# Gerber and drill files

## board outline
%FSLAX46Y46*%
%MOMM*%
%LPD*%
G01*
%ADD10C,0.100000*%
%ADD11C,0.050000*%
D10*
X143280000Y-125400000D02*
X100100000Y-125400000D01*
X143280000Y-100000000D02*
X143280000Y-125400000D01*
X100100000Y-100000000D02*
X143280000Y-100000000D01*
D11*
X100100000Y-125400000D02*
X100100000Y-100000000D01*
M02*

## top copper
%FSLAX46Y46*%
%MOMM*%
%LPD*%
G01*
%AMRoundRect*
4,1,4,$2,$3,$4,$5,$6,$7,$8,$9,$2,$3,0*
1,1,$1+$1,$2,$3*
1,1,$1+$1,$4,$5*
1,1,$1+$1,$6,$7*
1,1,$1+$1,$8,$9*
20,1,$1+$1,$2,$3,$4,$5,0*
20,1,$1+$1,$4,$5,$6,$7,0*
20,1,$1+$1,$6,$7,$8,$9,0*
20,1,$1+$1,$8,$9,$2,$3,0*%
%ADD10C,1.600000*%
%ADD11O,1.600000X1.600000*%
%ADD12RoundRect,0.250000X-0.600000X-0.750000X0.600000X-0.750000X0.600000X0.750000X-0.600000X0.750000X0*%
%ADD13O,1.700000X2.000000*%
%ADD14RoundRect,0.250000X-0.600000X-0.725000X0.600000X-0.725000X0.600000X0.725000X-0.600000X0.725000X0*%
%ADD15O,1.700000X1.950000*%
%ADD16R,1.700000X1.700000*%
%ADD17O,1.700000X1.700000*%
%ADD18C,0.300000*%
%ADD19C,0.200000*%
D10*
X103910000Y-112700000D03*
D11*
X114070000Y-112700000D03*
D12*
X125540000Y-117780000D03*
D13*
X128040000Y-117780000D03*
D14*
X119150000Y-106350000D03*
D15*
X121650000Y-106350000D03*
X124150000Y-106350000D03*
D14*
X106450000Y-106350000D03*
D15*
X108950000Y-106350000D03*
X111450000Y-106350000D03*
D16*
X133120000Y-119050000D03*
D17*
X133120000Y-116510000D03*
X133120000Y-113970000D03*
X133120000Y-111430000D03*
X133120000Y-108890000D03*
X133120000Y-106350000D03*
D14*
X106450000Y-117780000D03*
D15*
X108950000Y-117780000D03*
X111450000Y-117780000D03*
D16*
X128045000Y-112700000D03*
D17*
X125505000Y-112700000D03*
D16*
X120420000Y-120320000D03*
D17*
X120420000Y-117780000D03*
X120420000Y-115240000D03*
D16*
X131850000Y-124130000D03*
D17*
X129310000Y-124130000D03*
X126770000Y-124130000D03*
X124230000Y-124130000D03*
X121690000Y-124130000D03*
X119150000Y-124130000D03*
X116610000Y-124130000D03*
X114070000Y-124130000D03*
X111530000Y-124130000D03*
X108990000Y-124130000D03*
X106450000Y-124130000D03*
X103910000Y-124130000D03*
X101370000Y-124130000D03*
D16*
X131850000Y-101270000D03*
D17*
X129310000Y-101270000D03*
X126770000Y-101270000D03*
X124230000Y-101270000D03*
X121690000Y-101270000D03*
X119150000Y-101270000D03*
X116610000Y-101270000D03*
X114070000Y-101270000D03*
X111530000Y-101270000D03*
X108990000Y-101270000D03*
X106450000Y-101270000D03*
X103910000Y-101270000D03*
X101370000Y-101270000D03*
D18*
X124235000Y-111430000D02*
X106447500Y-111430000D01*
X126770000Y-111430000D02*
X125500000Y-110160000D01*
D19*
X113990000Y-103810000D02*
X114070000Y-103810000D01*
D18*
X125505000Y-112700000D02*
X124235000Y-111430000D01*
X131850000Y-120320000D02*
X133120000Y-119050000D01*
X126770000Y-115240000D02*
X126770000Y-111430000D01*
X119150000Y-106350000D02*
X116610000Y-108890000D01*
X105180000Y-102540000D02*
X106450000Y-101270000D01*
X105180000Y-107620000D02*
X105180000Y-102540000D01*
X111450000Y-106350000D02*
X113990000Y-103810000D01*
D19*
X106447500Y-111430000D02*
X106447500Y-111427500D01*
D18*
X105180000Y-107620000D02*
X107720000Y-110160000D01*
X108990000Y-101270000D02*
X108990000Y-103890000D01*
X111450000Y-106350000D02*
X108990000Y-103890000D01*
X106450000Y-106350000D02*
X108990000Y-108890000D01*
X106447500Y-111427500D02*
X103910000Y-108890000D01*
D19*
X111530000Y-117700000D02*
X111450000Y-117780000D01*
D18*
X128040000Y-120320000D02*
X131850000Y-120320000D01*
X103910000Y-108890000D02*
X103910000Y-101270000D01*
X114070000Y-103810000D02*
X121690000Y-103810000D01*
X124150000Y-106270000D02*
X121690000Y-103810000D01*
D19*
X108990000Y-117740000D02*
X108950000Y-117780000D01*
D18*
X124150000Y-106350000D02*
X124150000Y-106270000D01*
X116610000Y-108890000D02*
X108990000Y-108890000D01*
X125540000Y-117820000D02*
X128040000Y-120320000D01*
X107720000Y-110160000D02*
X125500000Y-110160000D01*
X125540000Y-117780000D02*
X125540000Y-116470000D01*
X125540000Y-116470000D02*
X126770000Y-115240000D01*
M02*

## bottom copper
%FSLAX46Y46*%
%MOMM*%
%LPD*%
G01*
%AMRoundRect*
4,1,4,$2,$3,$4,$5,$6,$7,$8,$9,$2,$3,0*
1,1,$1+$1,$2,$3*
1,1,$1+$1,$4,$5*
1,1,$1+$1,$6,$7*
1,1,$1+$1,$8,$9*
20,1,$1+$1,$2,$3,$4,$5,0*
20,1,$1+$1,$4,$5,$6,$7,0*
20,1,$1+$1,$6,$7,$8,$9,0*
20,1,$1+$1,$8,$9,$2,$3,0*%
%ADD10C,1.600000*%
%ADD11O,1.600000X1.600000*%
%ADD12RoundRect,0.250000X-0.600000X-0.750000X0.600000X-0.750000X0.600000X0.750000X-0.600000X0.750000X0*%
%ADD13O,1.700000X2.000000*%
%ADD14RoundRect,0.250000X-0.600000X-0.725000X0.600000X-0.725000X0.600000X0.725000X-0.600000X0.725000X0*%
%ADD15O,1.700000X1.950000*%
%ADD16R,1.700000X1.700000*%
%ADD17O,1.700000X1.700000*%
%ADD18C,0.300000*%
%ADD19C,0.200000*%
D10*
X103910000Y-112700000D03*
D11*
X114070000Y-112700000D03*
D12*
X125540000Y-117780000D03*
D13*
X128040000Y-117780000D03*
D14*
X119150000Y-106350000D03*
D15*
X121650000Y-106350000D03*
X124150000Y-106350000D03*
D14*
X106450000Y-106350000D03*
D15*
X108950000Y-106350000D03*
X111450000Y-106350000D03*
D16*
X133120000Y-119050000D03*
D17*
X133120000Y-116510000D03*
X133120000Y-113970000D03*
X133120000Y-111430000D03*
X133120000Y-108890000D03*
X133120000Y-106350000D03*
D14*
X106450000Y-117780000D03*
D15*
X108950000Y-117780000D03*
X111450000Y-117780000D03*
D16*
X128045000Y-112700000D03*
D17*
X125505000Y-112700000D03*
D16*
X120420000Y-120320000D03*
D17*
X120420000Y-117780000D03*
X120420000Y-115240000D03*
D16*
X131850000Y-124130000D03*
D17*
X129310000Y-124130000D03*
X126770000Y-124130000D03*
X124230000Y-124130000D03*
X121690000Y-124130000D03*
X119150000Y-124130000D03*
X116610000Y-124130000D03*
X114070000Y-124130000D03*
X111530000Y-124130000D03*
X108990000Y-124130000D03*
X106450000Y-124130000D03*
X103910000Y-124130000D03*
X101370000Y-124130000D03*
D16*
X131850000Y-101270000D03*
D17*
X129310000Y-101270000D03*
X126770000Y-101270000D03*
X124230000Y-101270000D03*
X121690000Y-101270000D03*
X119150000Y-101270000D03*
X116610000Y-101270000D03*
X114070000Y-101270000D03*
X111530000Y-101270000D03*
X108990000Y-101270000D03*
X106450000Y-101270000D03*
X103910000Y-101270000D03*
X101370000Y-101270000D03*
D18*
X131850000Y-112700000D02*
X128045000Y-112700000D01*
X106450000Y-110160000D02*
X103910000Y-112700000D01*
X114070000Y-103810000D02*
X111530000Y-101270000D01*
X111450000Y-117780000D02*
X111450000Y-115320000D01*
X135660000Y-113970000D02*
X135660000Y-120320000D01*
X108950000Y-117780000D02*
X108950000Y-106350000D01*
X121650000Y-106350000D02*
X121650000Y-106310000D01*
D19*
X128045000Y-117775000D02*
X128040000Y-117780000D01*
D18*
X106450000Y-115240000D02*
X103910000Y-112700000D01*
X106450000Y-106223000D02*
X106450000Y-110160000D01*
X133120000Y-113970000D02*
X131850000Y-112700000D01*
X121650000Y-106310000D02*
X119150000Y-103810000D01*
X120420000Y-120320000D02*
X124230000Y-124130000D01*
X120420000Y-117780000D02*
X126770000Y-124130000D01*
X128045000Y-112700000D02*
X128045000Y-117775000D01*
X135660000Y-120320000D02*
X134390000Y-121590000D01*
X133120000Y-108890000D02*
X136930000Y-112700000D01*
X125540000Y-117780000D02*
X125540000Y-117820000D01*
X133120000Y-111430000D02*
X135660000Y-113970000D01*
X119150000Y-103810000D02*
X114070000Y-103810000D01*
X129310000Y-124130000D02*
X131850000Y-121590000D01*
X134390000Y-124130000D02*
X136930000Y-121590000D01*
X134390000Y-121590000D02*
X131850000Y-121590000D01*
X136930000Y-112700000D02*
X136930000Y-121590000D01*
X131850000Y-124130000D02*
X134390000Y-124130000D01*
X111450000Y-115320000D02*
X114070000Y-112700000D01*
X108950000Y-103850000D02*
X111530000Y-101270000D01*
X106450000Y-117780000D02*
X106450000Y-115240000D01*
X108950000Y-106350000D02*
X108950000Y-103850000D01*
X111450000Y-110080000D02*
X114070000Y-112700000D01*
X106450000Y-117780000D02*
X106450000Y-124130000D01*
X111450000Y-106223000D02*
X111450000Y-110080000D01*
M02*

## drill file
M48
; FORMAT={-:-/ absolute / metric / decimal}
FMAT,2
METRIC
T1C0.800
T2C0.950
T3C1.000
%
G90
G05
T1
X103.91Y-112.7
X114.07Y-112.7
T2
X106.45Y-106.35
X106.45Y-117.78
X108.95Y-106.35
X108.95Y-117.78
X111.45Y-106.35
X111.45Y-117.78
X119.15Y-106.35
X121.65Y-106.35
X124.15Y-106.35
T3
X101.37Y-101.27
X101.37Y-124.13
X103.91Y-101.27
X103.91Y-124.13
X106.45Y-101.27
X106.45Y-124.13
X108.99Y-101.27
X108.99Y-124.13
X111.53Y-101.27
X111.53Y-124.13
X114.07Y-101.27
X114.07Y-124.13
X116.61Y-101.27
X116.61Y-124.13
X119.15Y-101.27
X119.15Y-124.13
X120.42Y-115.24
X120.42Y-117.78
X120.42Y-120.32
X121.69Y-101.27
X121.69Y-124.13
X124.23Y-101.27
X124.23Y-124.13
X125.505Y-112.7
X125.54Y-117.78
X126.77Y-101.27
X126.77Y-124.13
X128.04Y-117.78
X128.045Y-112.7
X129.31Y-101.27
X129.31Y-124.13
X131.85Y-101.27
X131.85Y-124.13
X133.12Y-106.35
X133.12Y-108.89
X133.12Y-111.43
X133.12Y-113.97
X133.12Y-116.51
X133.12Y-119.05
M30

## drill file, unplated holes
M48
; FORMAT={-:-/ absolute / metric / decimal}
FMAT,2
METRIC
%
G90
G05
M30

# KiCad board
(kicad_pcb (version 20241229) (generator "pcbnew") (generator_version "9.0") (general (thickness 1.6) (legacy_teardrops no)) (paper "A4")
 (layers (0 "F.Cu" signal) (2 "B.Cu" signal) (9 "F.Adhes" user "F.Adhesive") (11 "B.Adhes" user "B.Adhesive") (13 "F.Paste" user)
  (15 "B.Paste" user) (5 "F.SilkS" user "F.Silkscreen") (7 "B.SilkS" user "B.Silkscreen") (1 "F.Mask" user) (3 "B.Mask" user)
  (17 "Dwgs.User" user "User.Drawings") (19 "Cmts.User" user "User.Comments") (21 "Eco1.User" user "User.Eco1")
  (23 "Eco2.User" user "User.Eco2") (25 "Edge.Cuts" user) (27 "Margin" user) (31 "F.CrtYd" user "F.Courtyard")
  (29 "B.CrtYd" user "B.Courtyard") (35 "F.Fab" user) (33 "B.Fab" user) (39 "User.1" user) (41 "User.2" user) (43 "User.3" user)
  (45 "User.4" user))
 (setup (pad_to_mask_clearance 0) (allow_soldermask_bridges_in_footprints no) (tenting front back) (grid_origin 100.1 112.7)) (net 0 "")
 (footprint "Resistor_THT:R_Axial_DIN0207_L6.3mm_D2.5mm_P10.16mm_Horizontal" (layer "F.Cu") (at 103.91 112.7)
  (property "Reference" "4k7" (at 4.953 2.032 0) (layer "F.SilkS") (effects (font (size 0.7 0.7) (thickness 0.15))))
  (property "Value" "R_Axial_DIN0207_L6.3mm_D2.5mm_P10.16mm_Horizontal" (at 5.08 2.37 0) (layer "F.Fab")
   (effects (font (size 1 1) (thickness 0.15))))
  (pad "1" thru_hole circle (at 0 0) (size 1.6 1.6) (drill 0.8) (layers "*.Cu" "*.Mask") (remove_unused_layers no))
  (pad "2" thru_hole oval (at 10.16 0) (size 1.6 1.6) (drill 0.8) (layers "*.Cu" "*.Mask") (remove_unused_layers no)))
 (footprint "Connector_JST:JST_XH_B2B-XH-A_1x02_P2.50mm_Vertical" (layer "F.Cu") (at 125.54 117.78)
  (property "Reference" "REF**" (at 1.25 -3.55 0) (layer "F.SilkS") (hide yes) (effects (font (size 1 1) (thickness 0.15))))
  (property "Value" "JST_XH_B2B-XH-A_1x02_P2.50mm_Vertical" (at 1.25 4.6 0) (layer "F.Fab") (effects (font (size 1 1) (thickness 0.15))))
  (pad "1" thru_hole roundrect (at 0 0) (size 1.7 2) (drill 1) (layers "*.Cu" "*.Mask") (remove_unused_layers no)
   (roundrect_rratio 0.147059))
  (pad "2" thru_hole oval (at 2.5 0) (size 1.7 2) (drill 1) (layers "*.Cu" "*.Mask") (remove_unused_layers no)))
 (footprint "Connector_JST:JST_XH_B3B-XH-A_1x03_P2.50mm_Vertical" (layer "F.Cu") (at 119.15 106.35)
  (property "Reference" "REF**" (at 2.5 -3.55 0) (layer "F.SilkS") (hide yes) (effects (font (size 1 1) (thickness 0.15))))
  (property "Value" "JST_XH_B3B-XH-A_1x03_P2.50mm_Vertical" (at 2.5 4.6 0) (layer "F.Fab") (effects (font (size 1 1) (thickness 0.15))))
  (pad "1" thru_hole roundrect (at 0 0) (size 1.7 1.95) (drill 0.95) (layers "*.Cu" "*.Mask") (remove_unused_layers no)
   (roundrect_rratio 0.147059))
  (pad "2" thru_hole oval (at 2.5 0) (size 1.7 1.95) (drill 0.95) (layers "*.Cu" "*.Mask") (remove_unused_layers no))
  (pad "3" thru_hole oval (at 5 0) (size 1.7 1.95) (drill 0.95) (layers "*.Cu" "*.Mask") (remove_unused_layers no)))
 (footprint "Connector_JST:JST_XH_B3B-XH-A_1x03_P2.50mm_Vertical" (layer "F.Cu") (at 106.45 106.35)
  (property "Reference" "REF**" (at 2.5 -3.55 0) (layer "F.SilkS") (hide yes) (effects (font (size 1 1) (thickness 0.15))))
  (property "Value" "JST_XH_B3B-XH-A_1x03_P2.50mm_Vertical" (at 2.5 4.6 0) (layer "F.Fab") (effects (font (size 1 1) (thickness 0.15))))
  (pad "1" thru_hole roundrect (at 0 0) (size 1.7 1.95) (drill 0.95) (layers "*.Cu" "*.Mask") (remove_unused_layers no)
   (roundrect_rratio 0.147059))
  (pad "2" thru_hole oval (at 2.5 0) (size 1.7 1.95) (drill 0.95) (layers "*.Cu" "*.Mask") (remove_unused_layers no))
  (pad "3" thru_hole oval (at 5 0) (size 1.7 1.95) (drill 0.95) (layers "*.Cu" "*.Mask") (remove_unused_layers no)))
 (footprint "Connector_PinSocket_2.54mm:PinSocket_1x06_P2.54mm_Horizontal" (layer "F.Cu") (at 133.12 119.05 180)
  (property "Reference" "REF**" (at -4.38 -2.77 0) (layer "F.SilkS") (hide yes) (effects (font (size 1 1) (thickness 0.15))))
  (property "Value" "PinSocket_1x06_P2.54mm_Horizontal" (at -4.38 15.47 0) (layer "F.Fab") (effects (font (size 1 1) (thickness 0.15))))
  (pad "1" thru_hole rect (at 0 0 180) (size 1.7 1.7) (drill 1) (layers "*.Cu" "*.Mask") (remove_unused_layers no))
  (pad "2" thru_hole oval (at 0 2.54 180) (size 1.7 1.7) (drill 1) (layers "*.Cu" "*.Mask") (remove_unused_layers no))
  (pad "3" thru_hole oval (at 0 5.08 180) (size 1.7 1.7) (drill 1) (layers "*.Cu" "*.Mask") (remove_unused_layers no))
  (pad "4" thru_hole oval (at 0 7.62 180) (size 1.7 1.7) (drill 1) (layers "*.Cu" "*.Mask") (remove_unused_layers no))
  (pad "5" thru_hole oval (at 0 10.16 180) (size 1.7 1.7) (drill 1) (layers "*.Cu" "*.Mask") (remove_unused_layers no))
  (pad "6" thru_hole oval (at 0 12.7 180) (size 1.7 1.7) (drill 1) (layers "*.Cu" "*.Mask") (remove_unused_layers no)))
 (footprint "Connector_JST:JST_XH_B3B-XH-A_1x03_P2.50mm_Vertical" (layer "F.Cu") (at 106.45 117.78)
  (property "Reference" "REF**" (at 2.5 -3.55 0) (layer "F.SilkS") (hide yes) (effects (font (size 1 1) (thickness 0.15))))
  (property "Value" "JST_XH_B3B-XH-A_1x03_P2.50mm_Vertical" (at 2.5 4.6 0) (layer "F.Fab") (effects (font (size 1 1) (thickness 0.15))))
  (pad "1" thru_hole roundrect (at 0 0) (size 1.7 1.95) (drill 0.95) (layers "*.Cu" "*.Mask") (remove_unused_layers no)
   (roundrect_rratio 0.147059))
  (pad "2" thru_hole oval (at 2.5 0) (size 1.7 1.95) (drill 0.95) (layers "*.Cu" "*.Mask") (remove_unused_layers no))
  (pad "3" thru_hole oval (at 5 0) (size 1.7 1.95) (drill 0.95) (layers "*.Cu" "*.Mask") (remove_unused_layers no)))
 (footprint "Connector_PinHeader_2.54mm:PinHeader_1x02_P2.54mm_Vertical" (layer "F.Cu") (at 128.045 112.7 -90)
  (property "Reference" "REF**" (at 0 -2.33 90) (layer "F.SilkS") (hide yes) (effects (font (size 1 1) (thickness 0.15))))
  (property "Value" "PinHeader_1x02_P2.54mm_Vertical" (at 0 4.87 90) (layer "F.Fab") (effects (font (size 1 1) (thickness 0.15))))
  (pad "1" thru_hole rect (at 0 0 270) (size 1.7 1.7) (drill 1) (layers "*.Cu" "*.Mask") (remove_unused_layers no))
  (pad "2" thru_hole oval (at 0 2.54 270) (size 1.7 1.7) (drill 1) (layers "*.Cu" "*.Mask") (remove_unused_layers no)))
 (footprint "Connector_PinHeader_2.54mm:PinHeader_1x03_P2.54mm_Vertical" (layer "F.Cu") (at 120.42 120.32 180)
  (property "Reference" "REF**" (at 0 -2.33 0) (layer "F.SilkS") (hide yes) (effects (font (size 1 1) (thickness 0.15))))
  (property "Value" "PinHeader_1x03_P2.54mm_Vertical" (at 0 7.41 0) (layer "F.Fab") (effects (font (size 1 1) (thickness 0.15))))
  (pad "1" thru_hole rect (at 0 0 180) (size 1.7 1.7) (drill 1) (layers "*.Cu" "*.Mask") (remove_unused_layers no))
  (pad "2" thru_hole oval (at 0 2.54 180) (size 1.7 1.7) (drill 1) (layers "*.Cu" "*.Mask") (remove_unused_layers no))
  (pad "3" thru_hole oval (at 0 5.08 180) (size 1.7 1.7) (drill 1) (layers "*.Cu" "*.Mask") (remove_unused_layers no)))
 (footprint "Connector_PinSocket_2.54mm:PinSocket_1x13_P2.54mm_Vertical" (layer "B.Cu") (at 131.85 124.13 90)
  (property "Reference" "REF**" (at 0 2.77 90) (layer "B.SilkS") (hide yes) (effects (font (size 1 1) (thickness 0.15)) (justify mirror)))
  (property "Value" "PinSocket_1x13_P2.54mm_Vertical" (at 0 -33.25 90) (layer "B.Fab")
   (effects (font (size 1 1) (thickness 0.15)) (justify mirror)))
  (pad "1" thru_hole rect (at 0 0 90) (size 1.7 1.7) (drill 1) (layers "*.Cu" "*.Mask") (remove_unused_layers no))
  (pad "2" thru_hole oval (at 0 -2.54 90) (size 1.7 1.7) (drill 1) (layers "*.Cu" "*.Mask") (remove_unused_layers no))
  (pad "3" thru_hole oval (at 0 -5.08 90) (size 1.7 1.7) (drill 1) (layers "*.Cu" "*.Mask") (remove_unused_layers no))
  (pad "4" thru_hole oval (at 0 -7.62 90) (size 1.7 1.7) (drill 1) (layers "*.Cu" "*.Mask") (remove_unused_layers no))
  (pad "5" thru_hole oval (at 0 -10.16 90) (size 1.7 1.7) (drill 1) (layers "*.Cu" "*.Mask") (remove_unused_layers no))
  (pad "6" thru_hole oval (at 0 -12.7 90) (size 1.7 1.7) (drill 1) (layers "*.Cu" "*.Mask") (remove_unused_layers no))
  (pad "7" thru_hole oval (at 0 -15.24 90) (size 1.7 1.7) (drill 1) (layers "*.Cu" "*.Mask") (remove_unused_layers no))
  (pad "8" thru_hole oval (at 0 -17.78 90) (size 1.7 1.7) (drill 1) (layers "*.Cu" "*.Mask") (remove_unused_layers no))
  (pad "9" thru_hole oval (at 0 -20.32 90) (size 1.7 1.7) (drill 1) (layers "*.Cu" "*.Mask") (remove_unused_layers no))
  (pad "10" thru_hole oval (at 0 -22.86 90) (size 1.7 1.7) (drill 1) (layers "*.Cu" "*.Mask") (remove_unused_layers no))
  (pad "11" thru_hole oval (at 0 -25.4 90) (size 1.7 1.7) (drill 1) (layers "*.Cu" "*.Mask") (remove_unused_layers no))
  (pad "12" thru_hole oval (at 0 -27.94 90) (size 1.7 1.7) (drill 1) (layers "*.Cu" "*.Mask") (remove_unused_layers no))
  (pad "13" thru_hole oval (at 0 -30.48 90) (size 1.7 1.7) (drill 1) (layers "*.Cu" "*.Mask") (remove_unused_layers no)))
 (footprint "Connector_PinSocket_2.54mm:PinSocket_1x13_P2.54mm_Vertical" (layer "B.Cu") (at 131.85 101.27 90)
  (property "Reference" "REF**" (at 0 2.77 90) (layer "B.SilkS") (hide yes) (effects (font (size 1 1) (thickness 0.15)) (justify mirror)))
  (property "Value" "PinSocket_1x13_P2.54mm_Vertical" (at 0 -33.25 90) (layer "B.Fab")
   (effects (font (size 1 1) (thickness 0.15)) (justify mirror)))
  (pad "1" thru_hole rect (at 0 0 90) (size 1.7 1.7) (drill 1) (layers "*.Cu" "*.Mask") (remove_unused_layers no))
  (pad "2" thru_hole oval (at 0 -2.54 90) (size 1.7 1.7) (drill 1) (layers "*.Cu" "*.Mask") (remove_unused_layers no))
  (pad "3" thru_hole oval (at 0 -5.08 90) (size 1.7 1.7) (drill 1) (layers "*.Cu" "*.Mask") (remove_unused_layers no))
  (pad "4" thru_hole oval (at 0 -7.62 90) (size 1.7 1.7) (drill 1) (layers "*.Cu" "*.Mask") (remove_unused_layers no))
  (pad "5" thru_hole oval (at 0 -10.16 90) (size 1.7 1.7) (drill 1) (layers "*.Cu" "*.Mask") (remove_unused_layers no))
  (pad "6" thru_hole oval (at 0 -12.7 90) (size 1.7 1.7) (drill 1) (layers "*.Cu" "*.Mask") (remove_unused_layers no))
  (pad "7" thru_hole oval (at 0 -15.24 90) (size 1.7 1.7) (drill 1) (layers "*.Cu" "*.Mask") (remove_unused_layers no))
  (pad "8" thru_hole oval (at 0 -17.78 90) (size 1.7 1.7) (drill 1) (layers "*.Cu" "*.Mask") (remove_unused_layers no))
  (pad "9" thru_hole oval (at 0 -20.32 90) (size 1.7 1.7) (drill 1) (layers "*.Cu" "*.Mask") (remove_unused_layers no))
  (pad "10" thru_hole oval (at 0 -22.86 90) (size 1.7 1.7) (drill 1) (layers "*.Cu" "*.Mask") (remove_unused_layers no))
  (pad "11" thru_hole oval (at 0 -25.4 90) (size 1.7 1.7) (drill 1) (layers "*.Cu" "*.Mask") (remove_unused_layers no))
  (pad "12" thru_hole oval (at 0 -27.94 90) (size 1.7 1.7) (drill 1) (layers "*.Cu" "*.Mask") (remove_unused_layers no))
  (pad "13" thru_hole oval (at 0 -30.48 90) (size 1.7 1.7) (drill 1) (layers "*.Cu" "*.Mask") (remove_unused_layers no)))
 (gr_line (start 143.28 125.4) (end 100.1 125.4) (stroke (width 0.1) (type solid)) (layer "Edge.Cuts"))
 (gr_line (start 143.28 100) (end 143.28 125.4) (stroke (width 0.1) (type solid)) (layer "Edge.Cuts"))
 (gr_line (start 100.1 100) (end 143.28 100) (stroke (width 0.1) (type solid)) (layer "Edge.Cuts"))
 (gr_line (start 100.1 125.4) (end 100.1 100) (stroke (width 0.05) (type default)) (layer "Edge.Cuts"))
 (segment (start 124.235 111.43) (end 106.4475 111.43) (width 0.3) (layer "F.Cu") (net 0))
 (segment (start 126.77 111.43) (end 125.5 110.16) (width 0.3) (layer "F.Cu") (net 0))
 (segment (start 113.99 103.81) (end 114.07 103.81) (width 0.2) (layer "F.Cu") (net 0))
 (segment (start 125.505 112.7) (end 124.235 111.43) (width 0.3) (layer "F.Cu") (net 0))
 (segment (start 131.85 120.32) (end 133.12 119.05) (width 0.3) (layer "F.Cu") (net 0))
 (segment (start 126.77 115.24) (end 126.77 111.43) (width 0.3) (layer "F.Cu") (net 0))
 (segment (start 119.15 106.35) (end 116.61 108.89) (width 0.3) (layer "F.Cu") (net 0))
 (segment (start 105.18 102.54) (end 106.45 101.27) (width 0.3) (layer "F.Cu") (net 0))
 (segment (start 105.18 107.62) (end 105.18 102.54) (width 0.3) (layer "F.Cu") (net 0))
 (segment (start 111.45 106.35) (end 113.99 103.81) (width 0.3) (layer "F.Cu") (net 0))
 (segment (start 106.4475 111.43) (end 106.4475 111.4275) (width 0.2) (layer "F.Cu") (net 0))
 (segment (start 105.18 107.62) (end 107.72 110.16) (width 0.3) (layer "F.Cu") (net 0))
 (segment (start 108.99 101.27) (end 108.99 103.89) (width 0.3) (layer "F.Cu") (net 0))
 (segment (start 111.45 106.35) (end 108.99 103.89) (width 0.3) (layer "F.Cu") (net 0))
 (segment (start 106.45 106.35) (end 108.99 108.89) (width 0.3) (layer "F.Cu") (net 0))
 (segment (start 106.4475 111.4275) (end 103.91 108.89) (width 0.3) (layer "F.Cu") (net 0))
 (segment (start 111.53 117.7) (end 111.45 117.78) (width 0.2) (layer "F.Cu") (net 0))
 (segment (start 128.04 120.32) (end 131.85 120.32) (width 0.3) (layer "F.Cu") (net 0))
 (segment (start 103.91 108.89) (end 103.91 101.27) (width 0.3) (layer "F.Cu") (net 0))
 (segment (start 114.07 103.81) (end 121.69 103.81) (width 0.3) (layer "F.Cu") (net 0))
 (segment (start 124.15 106.27) (end 121.69 103.81) (width 0.3) (layer "F.Cu") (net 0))
 (segment (start 108.99 117.74) (end 108.95 117.78) (width 0.2) (layer "F.Cu") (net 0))
 (segment (start 124.15 106.35) (end 124.15 106.27) (width 0.3) (layer "F.Cu") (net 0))
 (segment (start 116.61 108.89) (end 108.99 108.89) (width 0.3) (layer "F.Cu") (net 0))
 (segment (start 125.54 117.82) (end 128.04 120.32) (width 0.3) (layer "F.Cu") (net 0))
 (segment (start 107.72 110.16) (end 125.5 110.16) (width 0.3) (layer "F.Cu") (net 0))
 (segment (start 125.54 117.78) (end 125.54 116.47) (width 0.3) (layer "F.Cu") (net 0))
 (segment (start 125.54 116.47) (end 126.77 115.24) (width 0.3) (layer "F.Cu") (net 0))
 (segment (start 131.85 112.7) (end 128.045 112.7) (width 0.3) (layer "B.Cu") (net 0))
 (segment (start 106.45 110.16) (end 103.91 112.7) (width 0.3) (layer "B.Cu") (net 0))
 (segment (start 114.07 103.81) (end 111.53 101.27) (width 0.3) (layer "B.Cu") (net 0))
 (segment (start 111.45 117.78) (end 111.45 115.32) (width 0.3) (layer "B.Cu") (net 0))
 (segment (start 135.66 113.97) (end 135.66 120.32) (width 0.3) (layer "B.Cu") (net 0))
 (segment (start 108.95 117.78) (end 108.95 106.35) (width 0.3) (layer "B.Cu") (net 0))
 (segment (start 121.65 106.35) (end 121.65 106.31) (width 0.3) (layer "B.Cu") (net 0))
 (segment (start 128.045 117.775) (end 128.04 117.78) (width 0.2) (layer "B.Cu") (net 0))
 (segment (start 106.45 115.24) (end 103.91 112.7) (width 0.3) (layer "B.Cu") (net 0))
 (segment (start 106.45 106.223) (end 106.45 110.16) (width 0.3) (layer "B.Cu") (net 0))
 (segment (start 133.12 113.97) (end 131.85 112.7) (width 0.3) (layer "B.Cu") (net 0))
 (segment (start 121.65 106.31) (end 119.15 103.81) (width 0.3) (layer "B.Cu") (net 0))
 (segment (start 120.42 120.32) (end 124.23 124.13) (width 0.3) (layer "B.Cu") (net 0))
 (segment (start 120.42 117.78) (end 126.77 124.13) (width 0.3) (layer "B.Cu") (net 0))
 (segment (start 128.045 112.7) (end 128.045 117.775) (width 0.3) (layer "B.Cu") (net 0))
 (segment (start 135.66 120.32) (end 134.39 121.59) (width 0.3) (layer "B.Cu") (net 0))
 (segment (start 133.12 108.89) (end 136.93 112.7) (width 0.3) (layer "B.Cu") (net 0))
 (segment (start 125.54 117.78) (end 125.54 117.82) (width 0.3) (layer "B.Cu") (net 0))
 (segment (start 133.12 111.43) (end 135.66 113.97) (width 0.3) (layer "B.Cu") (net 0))
 (segment (start 119.15 103.81) (end 114.07 103.81) (width 0.3) (layer "B.Cu") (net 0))
 (segment (start 129.31 124.13) (end 131.85 121.59) (width 0.3) (layer "B.Cu") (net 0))
 (segment (start 134.39 124.13) (end 136.93 121.59) (width 0.3) (layer "B.Cu") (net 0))
 (segment (start 134.39 121.59) (end 131.85 121.59) (width 0.3) (layer "B.Cu") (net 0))
 (segment (start 136.93 112.7) (end 136.93 121.59) (width 0.3) (layer "B.Cu") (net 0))
 (segment (start 131.85 124.13) (end 134.39 124.13) (width 0.3) (layer "B.Cu") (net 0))
 (segment (start 111.45 115.32) (end 114.07 112.7) (width 0.3) (layer "B.Cu") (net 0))
 (segment (start 108.95 103.85) (end 111.53 101.27) (width 0.3) (layer "B.Cu") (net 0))
 (segment (start 106.45 117.78) (end 106.45 115.24) (width 0.3) (layer "B.Cu") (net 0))
 (segment (start 108.95 106.35) (end 108.95 103.85) (width 0.3) (layer "B.Cu") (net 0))
 (segment (start 111.45 110.08) (end 114.07 112.7) (width 0.3) (layer "B.Cu") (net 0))
 (segment (start 106.45 117.78) (end 106.45 124.13) (width 0.3) (layer "B.Cu") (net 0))
 (segment (start 111.45 106.223) (end 111.45 110.08) (width 0.3) (layer "B.Cu") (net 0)))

